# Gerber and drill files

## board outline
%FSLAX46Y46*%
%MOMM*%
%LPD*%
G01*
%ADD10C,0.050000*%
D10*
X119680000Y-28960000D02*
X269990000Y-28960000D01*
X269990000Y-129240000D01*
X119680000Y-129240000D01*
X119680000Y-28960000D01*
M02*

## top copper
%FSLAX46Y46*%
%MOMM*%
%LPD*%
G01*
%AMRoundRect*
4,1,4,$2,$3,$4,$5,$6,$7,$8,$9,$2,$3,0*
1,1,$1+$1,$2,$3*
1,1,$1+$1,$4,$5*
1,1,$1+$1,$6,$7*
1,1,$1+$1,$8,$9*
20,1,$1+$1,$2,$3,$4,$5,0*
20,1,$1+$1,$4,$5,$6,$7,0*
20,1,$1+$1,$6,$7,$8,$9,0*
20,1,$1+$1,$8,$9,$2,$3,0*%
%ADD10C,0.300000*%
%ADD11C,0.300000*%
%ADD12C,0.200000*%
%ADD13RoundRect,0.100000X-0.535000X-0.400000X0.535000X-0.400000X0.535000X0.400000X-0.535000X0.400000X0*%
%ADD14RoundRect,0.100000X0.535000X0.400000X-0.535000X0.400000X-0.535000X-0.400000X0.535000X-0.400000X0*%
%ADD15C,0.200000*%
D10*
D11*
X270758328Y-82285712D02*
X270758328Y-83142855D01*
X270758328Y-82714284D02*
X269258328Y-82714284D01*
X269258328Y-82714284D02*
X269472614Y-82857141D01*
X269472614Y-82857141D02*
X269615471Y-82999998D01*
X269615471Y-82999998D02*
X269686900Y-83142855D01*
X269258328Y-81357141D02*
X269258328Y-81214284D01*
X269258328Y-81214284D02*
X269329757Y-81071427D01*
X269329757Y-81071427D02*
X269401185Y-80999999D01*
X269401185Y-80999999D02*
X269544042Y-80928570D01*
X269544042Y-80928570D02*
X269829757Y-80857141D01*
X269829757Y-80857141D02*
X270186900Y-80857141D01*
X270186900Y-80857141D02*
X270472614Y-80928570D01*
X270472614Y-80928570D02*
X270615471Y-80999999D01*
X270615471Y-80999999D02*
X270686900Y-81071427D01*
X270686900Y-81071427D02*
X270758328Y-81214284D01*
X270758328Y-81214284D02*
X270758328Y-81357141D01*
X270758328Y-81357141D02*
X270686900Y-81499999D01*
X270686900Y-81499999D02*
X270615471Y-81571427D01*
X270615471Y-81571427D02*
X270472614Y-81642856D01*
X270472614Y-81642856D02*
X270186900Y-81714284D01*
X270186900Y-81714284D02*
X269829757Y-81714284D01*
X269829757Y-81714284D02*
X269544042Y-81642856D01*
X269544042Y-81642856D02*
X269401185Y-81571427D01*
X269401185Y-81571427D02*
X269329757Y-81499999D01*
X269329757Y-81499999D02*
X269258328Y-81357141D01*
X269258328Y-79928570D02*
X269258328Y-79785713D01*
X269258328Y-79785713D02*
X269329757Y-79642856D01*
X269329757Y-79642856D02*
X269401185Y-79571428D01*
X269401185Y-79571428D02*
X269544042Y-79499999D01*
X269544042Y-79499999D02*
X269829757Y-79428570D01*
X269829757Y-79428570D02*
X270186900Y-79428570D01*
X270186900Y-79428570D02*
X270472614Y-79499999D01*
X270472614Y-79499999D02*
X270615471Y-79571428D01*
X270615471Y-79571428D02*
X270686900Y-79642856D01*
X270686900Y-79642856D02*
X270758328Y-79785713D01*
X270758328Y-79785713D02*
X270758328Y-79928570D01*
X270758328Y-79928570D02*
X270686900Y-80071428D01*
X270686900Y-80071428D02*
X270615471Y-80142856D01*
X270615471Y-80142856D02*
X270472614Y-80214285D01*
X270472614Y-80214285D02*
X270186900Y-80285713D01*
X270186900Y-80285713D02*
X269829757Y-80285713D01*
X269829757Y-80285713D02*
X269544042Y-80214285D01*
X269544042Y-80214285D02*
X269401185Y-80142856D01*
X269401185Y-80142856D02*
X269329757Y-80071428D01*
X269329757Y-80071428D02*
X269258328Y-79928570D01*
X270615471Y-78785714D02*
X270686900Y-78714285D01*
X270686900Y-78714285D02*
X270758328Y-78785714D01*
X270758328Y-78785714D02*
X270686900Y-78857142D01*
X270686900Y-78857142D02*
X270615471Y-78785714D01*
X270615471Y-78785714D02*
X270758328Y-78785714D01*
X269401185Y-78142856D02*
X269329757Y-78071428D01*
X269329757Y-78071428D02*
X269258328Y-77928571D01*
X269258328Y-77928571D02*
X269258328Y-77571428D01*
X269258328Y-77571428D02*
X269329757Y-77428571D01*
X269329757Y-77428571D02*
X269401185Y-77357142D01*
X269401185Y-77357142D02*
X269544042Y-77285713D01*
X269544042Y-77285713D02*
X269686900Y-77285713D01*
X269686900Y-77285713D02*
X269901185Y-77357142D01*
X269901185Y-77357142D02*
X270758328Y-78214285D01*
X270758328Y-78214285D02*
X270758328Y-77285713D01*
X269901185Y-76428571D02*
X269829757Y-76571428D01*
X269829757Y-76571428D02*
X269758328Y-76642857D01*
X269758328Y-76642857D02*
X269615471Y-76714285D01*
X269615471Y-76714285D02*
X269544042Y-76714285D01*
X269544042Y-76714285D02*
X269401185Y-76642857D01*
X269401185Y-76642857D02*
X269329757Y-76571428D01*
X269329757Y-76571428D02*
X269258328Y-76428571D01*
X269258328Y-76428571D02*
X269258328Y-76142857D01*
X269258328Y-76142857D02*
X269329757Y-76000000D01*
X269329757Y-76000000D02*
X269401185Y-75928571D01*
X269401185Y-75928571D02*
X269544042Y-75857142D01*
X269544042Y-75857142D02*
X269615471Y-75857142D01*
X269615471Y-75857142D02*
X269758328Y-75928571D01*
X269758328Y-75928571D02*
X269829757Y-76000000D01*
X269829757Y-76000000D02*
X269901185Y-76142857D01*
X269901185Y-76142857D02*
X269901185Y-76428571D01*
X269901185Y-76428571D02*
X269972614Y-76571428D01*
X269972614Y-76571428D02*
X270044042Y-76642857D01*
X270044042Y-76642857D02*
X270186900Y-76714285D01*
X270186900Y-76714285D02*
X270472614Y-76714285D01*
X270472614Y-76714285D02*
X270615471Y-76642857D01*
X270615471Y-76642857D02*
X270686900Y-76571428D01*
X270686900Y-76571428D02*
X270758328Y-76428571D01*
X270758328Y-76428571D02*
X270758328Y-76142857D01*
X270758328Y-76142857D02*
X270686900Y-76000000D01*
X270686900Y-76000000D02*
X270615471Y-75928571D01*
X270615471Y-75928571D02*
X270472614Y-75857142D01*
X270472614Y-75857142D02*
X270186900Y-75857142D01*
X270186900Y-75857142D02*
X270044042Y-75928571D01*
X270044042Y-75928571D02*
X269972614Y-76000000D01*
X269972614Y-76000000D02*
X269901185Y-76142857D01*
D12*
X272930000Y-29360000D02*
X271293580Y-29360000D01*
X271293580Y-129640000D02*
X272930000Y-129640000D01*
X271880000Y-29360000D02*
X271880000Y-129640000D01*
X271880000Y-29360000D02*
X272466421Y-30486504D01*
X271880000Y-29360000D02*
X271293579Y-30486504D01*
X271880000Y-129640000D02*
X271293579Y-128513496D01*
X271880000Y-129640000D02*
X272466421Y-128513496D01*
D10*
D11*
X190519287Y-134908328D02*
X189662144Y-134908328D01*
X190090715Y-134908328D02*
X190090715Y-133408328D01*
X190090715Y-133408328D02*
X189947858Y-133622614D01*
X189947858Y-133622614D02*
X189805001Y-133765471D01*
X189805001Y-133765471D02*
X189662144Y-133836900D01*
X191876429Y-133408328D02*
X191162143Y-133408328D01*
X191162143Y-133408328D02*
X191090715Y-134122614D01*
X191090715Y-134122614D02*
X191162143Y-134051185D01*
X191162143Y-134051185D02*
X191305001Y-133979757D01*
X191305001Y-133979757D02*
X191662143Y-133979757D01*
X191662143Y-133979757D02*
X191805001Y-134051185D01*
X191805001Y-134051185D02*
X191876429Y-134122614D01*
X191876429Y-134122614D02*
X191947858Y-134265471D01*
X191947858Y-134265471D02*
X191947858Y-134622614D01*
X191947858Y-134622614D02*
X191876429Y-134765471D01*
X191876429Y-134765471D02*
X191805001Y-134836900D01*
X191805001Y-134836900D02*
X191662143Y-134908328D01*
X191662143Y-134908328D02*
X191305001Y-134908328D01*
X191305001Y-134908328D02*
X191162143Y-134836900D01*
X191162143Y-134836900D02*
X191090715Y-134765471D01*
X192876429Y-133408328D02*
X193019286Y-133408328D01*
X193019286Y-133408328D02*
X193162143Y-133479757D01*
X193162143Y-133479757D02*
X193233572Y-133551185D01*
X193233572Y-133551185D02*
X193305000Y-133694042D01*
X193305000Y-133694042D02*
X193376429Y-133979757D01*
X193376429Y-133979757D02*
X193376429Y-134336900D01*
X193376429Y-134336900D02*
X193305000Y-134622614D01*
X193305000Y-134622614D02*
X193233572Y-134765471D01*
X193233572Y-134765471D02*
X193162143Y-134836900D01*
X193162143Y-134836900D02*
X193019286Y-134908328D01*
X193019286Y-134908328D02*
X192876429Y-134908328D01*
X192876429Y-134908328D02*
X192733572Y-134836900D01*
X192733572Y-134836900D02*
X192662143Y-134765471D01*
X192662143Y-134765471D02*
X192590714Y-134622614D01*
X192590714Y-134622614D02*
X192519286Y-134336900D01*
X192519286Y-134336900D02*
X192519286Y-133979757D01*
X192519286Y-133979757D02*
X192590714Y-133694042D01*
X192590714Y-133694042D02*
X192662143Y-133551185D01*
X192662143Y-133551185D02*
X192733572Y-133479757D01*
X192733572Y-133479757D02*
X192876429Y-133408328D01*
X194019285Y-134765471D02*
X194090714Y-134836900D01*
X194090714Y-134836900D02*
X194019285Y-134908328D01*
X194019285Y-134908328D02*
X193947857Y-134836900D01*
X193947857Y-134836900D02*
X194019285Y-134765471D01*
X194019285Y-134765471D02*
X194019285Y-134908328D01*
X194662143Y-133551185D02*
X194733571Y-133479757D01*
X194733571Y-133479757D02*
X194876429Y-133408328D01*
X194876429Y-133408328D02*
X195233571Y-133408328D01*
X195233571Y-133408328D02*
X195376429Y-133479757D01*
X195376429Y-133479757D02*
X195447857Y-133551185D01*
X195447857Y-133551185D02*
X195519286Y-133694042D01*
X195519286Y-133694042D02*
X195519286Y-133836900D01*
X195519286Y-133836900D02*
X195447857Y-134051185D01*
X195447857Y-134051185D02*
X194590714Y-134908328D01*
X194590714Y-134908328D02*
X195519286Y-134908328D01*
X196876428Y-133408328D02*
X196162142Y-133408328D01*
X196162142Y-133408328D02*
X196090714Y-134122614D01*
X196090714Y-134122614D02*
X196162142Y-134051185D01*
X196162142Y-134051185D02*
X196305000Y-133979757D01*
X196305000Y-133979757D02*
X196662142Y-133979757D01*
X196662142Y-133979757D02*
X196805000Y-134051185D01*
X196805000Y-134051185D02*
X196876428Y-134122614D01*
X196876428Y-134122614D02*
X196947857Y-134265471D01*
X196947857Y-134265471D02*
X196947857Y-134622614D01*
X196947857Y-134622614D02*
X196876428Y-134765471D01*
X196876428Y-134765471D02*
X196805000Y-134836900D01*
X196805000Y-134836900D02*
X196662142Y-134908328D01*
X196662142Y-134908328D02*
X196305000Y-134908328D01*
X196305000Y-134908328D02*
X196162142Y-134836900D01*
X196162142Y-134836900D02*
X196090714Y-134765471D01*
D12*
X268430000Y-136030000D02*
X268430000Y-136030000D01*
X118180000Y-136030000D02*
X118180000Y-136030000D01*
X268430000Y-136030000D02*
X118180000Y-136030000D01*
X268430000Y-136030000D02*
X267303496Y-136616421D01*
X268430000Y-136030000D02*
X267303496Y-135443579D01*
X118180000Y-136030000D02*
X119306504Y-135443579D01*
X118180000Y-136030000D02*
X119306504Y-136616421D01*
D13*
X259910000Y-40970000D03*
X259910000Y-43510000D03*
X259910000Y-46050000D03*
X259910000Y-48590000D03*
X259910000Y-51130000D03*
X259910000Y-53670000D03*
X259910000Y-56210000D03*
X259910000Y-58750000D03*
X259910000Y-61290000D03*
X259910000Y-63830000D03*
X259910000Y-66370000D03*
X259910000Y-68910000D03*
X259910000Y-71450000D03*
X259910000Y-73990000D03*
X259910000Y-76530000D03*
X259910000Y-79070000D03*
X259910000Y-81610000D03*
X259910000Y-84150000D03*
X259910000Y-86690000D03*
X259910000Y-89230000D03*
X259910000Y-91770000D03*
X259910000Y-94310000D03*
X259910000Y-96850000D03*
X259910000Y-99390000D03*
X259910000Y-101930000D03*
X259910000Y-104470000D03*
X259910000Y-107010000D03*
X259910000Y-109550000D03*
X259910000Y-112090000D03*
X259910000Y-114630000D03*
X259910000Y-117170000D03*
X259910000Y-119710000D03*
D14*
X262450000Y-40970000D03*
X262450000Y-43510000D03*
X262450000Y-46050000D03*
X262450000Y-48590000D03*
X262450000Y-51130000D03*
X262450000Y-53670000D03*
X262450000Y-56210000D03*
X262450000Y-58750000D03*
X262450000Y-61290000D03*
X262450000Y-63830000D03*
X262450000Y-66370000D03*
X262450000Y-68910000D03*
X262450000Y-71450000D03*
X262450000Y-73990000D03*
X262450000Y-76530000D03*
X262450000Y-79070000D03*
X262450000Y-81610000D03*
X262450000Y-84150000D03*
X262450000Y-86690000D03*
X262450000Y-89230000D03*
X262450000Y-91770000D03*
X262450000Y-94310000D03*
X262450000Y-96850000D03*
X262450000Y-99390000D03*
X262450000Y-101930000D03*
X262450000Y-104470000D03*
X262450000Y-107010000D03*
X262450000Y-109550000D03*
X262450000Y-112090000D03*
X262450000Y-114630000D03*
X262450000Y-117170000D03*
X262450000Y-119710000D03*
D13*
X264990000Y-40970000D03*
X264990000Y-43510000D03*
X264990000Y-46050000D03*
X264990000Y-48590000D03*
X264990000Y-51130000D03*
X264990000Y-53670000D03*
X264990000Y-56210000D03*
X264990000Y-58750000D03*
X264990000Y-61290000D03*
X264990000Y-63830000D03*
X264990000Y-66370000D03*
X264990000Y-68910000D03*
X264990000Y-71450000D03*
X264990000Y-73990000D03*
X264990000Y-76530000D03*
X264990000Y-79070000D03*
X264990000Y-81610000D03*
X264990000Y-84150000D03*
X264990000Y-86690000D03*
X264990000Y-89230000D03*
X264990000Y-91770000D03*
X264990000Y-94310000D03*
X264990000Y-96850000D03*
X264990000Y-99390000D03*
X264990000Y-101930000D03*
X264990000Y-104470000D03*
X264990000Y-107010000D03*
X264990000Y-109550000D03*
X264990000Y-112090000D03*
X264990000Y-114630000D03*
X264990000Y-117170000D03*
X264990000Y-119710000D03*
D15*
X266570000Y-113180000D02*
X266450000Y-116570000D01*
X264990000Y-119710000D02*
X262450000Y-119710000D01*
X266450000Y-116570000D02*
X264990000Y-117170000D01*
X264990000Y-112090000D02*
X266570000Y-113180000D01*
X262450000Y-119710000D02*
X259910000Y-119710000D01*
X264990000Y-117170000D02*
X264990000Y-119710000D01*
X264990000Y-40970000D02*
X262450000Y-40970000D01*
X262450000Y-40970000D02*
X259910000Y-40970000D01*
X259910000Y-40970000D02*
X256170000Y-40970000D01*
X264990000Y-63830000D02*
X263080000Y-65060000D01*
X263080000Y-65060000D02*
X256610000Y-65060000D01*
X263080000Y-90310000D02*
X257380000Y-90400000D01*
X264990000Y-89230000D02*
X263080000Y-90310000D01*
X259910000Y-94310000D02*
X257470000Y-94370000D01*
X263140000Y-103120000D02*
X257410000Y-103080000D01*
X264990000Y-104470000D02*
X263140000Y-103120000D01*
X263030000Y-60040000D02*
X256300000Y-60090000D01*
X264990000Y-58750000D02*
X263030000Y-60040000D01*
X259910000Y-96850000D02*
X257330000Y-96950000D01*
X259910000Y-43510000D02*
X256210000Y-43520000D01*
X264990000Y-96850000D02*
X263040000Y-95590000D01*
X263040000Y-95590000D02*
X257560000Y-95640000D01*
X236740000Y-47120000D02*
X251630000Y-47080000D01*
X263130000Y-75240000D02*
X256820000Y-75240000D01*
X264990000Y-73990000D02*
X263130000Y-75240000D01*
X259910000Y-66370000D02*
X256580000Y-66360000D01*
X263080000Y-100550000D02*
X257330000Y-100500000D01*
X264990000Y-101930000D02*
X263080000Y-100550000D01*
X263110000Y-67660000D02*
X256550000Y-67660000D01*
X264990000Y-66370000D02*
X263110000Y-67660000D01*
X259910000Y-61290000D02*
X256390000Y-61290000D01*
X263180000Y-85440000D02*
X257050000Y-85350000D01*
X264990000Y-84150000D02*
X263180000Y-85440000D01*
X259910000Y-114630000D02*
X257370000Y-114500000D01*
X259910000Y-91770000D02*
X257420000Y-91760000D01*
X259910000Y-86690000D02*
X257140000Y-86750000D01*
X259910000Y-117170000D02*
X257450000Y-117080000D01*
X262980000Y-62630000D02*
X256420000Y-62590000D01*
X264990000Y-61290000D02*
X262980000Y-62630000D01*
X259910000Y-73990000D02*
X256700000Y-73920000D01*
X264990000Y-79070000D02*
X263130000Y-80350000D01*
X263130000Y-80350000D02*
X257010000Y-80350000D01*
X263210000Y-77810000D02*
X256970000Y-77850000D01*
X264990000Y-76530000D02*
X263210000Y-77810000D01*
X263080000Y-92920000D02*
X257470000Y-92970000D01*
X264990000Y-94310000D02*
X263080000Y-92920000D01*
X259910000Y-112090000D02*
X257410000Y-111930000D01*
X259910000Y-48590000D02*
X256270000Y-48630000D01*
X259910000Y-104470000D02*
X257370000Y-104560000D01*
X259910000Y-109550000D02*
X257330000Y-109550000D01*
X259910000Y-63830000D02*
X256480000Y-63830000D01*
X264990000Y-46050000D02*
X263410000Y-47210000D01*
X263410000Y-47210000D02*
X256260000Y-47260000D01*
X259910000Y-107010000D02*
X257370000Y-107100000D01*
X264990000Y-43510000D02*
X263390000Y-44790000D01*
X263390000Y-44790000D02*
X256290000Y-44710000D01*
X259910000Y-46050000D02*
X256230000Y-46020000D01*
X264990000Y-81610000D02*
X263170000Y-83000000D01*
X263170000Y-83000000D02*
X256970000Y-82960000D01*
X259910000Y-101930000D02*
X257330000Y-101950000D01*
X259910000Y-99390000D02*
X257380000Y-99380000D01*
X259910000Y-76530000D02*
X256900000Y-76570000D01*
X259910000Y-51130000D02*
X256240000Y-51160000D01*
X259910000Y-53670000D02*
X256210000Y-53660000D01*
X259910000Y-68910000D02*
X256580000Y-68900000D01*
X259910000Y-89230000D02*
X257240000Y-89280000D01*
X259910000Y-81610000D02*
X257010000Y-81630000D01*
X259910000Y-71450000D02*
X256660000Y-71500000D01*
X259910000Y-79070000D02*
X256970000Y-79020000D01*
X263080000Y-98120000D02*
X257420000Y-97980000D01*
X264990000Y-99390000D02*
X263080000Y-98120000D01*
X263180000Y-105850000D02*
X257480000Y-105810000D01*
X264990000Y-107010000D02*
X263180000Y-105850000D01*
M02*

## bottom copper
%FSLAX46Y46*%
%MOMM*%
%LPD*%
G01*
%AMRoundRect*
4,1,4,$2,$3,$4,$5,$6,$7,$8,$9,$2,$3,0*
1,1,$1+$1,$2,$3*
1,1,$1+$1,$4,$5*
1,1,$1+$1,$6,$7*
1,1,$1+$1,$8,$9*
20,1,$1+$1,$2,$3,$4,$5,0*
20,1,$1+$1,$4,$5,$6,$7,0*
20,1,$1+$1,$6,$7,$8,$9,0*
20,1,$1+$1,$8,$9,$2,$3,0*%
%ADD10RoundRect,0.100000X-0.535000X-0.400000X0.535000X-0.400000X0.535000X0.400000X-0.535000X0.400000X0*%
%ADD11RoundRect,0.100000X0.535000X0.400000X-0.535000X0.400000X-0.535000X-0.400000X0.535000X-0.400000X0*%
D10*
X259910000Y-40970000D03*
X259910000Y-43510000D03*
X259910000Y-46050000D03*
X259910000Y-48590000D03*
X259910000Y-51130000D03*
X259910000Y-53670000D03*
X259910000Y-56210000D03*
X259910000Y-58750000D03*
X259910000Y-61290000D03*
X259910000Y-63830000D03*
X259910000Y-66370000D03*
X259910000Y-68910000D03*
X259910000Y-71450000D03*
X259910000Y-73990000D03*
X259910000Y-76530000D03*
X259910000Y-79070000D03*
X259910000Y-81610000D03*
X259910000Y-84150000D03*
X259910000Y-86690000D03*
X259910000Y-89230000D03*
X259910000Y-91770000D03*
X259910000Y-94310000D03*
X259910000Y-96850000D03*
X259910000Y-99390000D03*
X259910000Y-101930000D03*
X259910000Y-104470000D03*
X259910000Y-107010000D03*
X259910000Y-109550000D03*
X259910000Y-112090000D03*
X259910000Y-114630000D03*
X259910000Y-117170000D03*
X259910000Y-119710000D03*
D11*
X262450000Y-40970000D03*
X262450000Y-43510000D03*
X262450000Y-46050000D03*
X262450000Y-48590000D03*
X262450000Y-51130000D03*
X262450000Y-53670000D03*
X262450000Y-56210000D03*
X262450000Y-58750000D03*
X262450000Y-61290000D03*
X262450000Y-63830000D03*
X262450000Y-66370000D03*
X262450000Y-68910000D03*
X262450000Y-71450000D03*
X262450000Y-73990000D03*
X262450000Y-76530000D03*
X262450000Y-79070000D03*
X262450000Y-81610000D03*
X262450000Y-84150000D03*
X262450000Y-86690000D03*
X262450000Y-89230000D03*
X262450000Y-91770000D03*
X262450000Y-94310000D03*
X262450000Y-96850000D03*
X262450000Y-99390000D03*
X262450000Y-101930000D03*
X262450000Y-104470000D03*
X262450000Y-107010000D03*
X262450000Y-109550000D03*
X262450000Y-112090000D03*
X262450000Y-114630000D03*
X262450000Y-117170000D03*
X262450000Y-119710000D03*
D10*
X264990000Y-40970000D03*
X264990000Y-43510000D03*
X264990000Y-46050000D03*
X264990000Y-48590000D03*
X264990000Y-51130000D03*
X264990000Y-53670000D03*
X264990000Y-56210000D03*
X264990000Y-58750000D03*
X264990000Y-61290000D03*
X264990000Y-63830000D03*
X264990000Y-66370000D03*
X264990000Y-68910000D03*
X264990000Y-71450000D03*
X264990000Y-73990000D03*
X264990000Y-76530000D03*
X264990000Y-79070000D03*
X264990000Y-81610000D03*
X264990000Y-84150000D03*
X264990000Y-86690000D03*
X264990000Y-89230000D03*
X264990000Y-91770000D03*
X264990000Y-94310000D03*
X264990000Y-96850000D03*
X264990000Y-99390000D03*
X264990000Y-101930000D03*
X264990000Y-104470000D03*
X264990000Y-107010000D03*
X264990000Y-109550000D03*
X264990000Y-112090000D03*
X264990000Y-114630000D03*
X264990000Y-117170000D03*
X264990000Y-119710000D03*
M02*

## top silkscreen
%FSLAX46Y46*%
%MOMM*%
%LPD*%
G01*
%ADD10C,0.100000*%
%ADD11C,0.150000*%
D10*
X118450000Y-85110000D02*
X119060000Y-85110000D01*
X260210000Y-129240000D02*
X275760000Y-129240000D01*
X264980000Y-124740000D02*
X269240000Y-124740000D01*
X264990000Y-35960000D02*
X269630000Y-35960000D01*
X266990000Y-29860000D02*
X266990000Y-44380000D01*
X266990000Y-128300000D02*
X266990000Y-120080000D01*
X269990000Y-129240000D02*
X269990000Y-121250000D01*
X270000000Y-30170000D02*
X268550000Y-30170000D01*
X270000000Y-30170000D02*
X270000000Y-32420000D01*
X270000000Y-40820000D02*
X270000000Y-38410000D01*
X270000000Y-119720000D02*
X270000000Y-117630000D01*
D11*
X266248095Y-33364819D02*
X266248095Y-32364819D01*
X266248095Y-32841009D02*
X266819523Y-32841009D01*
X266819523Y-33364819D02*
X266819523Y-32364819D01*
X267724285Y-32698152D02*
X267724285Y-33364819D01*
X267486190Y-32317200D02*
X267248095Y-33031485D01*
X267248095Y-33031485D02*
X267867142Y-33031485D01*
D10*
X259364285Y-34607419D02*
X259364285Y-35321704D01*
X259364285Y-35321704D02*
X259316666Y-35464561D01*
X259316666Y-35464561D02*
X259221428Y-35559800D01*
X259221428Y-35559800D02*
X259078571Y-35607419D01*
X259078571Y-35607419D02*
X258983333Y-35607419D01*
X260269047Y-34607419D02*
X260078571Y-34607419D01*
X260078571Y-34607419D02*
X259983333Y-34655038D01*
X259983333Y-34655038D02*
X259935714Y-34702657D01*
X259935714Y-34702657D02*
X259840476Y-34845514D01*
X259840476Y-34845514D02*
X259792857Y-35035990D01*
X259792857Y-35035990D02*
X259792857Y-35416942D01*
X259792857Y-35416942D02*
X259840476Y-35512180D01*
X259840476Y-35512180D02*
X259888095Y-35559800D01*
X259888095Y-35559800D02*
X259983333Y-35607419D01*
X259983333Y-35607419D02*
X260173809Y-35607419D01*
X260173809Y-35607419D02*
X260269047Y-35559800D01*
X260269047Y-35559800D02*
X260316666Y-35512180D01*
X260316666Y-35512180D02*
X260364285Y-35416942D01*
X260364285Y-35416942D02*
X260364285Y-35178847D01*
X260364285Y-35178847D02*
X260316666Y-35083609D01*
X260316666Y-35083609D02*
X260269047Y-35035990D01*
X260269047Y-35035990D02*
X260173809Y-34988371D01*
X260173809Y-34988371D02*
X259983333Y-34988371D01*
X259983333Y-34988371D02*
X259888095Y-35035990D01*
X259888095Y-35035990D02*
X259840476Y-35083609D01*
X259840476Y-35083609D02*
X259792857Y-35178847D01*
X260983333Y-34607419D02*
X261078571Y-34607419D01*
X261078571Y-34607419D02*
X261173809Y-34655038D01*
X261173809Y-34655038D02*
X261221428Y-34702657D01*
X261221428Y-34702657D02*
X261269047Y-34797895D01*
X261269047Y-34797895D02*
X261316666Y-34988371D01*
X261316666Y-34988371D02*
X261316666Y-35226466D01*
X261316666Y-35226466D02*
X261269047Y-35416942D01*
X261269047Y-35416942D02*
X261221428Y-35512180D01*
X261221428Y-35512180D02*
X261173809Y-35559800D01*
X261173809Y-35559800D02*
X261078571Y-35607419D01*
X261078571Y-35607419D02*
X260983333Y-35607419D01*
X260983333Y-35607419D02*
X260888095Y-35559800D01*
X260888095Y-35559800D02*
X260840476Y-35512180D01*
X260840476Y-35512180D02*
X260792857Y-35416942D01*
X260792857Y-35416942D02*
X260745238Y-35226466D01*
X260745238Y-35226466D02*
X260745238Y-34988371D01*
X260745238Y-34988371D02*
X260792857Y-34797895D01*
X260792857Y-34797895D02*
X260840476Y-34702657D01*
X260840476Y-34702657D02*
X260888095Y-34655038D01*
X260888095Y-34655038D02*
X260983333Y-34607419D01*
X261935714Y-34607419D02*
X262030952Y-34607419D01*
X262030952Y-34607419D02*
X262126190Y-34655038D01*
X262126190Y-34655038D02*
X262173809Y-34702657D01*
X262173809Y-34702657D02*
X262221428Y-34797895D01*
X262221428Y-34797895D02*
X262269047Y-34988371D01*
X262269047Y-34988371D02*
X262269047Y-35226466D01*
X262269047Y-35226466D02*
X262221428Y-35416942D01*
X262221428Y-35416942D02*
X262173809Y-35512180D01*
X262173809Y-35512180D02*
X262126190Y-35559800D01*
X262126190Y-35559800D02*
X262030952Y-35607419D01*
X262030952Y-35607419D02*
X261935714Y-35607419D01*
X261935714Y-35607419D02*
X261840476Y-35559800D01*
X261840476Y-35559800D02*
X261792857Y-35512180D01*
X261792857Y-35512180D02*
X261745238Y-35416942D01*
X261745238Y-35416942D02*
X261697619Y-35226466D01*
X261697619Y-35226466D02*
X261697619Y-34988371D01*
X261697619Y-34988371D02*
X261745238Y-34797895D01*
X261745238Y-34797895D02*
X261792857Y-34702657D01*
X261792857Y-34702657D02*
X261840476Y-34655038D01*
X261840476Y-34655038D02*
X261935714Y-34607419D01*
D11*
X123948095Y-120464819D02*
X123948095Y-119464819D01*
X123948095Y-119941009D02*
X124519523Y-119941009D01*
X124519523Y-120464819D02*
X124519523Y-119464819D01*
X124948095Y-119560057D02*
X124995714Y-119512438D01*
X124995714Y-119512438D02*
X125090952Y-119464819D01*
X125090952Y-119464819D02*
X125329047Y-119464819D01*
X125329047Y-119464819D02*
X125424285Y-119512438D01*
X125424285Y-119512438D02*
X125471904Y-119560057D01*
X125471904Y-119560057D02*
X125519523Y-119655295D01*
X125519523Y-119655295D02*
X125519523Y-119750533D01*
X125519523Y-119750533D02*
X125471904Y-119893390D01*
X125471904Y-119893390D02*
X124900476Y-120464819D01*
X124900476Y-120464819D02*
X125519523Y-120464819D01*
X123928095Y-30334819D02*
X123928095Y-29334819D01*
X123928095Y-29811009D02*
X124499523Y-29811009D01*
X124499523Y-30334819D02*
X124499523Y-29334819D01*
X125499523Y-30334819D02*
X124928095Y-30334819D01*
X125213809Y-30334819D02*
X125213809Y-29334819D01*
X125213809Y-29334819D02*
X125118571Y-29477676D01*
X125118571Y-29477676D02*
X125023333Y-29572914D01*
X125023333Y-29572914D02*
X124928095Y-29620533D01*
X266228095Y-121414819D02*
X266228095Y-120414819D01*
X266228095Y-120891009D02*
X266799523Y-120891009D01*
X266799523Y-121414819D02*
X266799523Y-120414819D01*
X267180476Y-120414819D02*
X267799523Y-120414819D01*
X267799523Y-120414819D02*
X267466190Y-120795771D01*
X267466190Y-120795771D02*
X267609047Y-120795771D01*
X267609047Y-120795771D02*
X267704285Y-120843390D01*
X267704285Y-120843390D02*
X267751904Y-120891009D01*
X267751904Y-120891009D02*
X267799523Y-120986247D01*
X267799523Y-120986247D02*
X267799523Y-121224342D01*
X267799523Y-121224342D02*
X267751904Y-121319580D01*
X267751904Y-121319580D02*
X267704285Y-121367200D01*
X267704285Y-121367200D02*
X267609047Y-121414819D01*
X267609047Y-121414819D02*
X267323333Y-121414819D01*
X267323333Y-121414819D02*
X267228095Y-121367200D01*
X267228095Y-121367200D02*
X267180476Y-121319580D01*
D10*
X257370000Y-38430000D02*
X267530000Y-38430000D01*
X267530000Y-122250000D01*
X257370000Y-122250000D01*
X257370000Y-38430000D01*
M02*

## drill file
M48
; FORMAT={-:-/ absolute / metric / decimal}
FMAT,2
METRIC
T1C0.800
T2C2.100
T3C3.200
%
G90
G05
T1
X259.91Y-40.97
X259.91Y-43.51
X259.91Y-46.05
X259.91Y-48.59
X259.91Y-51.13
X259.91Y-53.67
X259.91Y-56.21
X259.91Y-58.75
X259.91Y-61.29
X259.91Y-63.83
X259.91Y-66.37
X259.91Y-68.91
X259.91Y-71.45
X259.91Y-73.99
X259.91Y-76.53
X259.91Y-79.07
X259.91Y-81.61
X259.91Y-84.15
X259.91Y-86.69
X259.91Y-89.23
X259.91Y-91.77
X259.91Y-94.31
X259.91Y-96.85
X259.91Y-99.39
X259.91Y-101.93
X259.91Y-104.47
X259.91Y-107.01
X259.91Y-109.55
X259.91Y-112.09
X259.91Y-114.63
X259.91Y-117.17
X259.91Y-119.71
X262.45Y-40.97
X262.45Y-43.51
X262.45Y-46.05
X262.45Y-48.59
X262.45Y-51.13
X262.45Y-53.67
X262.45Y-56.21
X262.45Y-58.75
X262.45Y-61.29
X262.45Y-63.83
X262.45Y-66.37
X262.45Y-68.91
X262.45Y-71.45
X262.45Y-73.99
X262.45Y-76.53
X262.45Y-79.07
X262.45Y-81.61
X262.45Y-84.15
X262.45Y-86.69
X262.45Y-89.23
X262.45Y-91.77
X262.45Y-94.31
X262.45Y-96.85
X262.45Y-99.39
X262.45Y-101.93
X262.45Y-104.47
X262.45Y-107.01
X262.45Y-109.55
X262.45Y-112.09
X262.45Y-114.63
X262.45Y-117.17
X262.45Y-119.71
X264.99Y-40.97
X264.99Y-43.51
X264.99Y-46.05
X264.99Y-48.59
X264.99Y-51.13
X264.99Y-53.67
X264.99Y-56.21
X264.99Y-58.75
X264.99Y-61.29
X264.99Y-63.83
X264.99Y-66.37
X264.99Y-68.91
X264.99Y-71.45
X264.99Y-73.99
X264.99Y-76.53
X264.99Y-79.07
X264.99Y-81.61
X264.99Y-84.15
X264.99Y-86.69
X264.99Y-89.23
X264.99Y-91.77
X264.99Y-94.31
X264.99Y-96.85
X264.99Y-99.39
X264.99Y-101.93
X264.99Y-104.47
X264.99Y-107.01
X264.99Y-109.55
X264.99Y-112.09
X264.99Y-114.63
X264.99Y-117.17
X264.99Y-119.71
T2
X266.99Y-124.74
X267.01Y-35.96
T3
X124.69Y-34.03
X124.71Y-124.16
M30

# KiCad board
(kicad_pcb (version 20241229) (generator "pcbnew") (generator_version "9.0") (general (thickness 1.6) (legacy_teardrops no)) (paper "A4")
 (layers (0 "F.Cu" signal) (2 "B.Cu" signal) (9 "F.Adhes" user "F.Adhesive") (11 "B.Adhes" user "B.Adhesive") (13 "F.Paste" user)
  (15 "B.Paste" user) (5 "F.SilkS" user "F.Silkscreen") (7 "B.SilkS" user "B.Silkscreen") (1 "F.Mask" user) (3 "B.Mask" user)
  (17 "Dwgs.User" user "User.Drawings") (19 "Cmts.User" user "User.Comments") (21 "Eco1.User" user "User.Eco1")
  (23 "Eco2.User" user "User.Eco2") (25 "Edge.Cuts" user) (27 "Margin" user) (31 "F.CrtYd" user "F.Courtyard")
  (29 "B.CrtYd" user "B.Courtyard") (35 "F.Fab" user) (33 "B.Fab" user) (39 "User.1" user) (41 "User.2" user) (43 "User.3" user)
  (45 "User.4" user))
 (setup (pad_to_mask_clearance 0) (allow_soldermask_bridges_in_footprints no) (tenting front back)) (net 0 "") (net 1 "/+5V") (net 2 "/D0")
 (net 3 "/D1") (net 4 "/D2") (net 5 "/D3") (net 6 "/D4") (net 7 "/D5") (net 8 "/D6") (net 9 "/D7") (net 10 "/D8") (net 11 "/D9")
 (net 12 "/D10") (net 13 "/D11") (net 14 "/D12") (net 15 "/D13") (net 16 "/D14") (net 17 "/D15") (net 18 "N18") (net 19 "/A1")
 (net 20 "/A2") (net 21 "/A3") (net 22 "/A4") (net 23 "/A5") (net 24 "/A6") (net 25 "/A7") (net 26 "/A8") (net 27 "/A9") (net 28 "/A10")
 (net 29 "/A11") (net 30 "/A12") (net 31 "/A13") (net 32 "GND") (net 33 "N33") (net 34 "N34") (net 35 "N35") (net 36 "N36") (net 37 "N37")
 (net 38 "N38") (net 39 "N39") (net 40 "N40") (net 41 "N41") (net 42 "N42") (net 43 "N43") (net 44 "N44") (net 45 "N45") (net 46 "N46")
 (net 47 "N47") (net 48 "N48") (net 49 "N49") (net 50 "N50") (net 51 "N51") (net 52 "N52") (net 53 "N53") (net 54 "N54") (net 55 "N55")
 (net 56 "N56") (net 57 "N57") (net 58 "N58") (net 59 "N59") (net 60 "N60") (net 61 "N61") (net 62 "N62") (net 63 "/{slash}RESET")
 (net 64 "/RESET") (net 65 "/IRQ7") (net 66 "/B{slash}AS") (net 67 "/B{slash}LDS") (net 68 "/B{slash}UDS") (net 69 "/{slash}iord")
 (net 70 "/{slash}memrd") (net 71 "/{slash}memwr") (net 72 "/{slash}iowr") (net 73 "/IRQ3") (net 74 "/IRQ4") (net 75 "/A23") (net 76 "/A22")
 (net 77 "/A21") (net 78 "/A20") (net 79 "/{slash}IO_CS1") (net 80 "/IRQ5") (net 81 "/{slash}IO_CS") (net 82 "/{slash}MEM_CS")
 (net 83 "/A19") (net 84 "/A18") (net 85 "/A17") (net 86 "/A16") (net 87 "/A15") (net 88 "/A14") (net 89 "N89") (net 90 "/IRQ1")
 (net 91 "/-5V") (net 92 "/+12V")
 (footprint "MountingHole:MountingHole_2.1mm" (layer "F.Cu") (at 267.01 35.96)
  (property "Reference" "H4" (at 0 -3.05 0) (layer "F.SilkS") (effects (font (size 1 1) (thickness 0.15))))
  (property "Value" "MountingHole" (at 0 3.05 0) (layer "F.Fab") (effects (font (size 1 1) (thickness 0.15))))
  (pad "" np_thru_hole circle (at 0 0) (size 2.1 2.1) (drill 2.1) (layers "*.Cu" "*.Mask")))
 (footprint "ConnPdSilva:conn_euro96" (layer "F.Cu") (at 262.45 35.89)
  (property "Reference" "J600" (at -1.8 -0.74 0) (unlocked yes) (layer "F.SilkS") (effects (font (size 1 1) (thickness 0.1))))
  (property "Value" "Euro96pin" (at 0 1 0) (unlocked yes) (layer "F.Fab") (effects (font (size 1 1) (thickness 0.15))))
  (fp_rect (start -5.08 2.54) (end 5.08 86.36) (stroke (width 0.1) (type default)) (fill no) (layer "F.SilkS"))
  (pad "1" thru_hole roundrect (at -2.54 5.08) (size 1.27 1) (drill 0.8) (layers "*.Cu" "*.Mask") (remove_unused_layers no)
   (roundrect_rratio 0.1) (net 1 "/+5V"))
  (pad "2" thru_hole roundrect (at -2.54 7.62) (size 1.27 1) (drill 0.8) (layers "*.Cu" "*.Mask") (remove_unused_layers no)
   (roundrect_rratio 0.1) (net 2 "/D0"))
  (pad "3" thru_hole roundrect (at -2.54 10.16) (size 1.27 1) (drill 0.8) (layers "*.Cu" "*.Mask") (remove_unused_layers no)
   (roundrect_rratio 0.1) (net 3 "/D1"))
  (pad "4" thru_hole roundrect (at -2.54 12.7) (size 1.27 1) (drill 0.8) (layers "*.Cu" "*.Mask") (remove_unused_layers no)
   (roundrect_rratio 0.1) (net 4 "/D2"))
  (pad "5" thru_hole roundrect (at -2.54 15.24) (size 1.27 1) (drill 0.8) (layers "*.Cu" "*.Mask") (remove_unused_layers no)
   (roundrect_rratio 0.1) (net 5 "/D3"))
  (pad "6" thru_hole roundrect (at -2.54 17.78) (size 1.27 1) (drill 0.8) (layers "*.Cu" "*.Mask") (remove_unused_layers no)
   (roundrect_rratio 0.1) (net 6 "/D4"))
  (pad "7" thru_hole roundrect (at -2.54 20.32) (size 1.27 1) (drill 0.8) (layers "*.Cu" "*.Mask") (remove_unused_layers no)
   (roundrect_rratio 0.1) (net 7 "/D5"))
  (pad "8" thru_hole roundrect (at -2.54 22.86) (size 1.27 1) (drill 0.8) (layers "*.Cu" "*.Mask") (remove_unused_layers no)
   (roundrect_rratio 0.1) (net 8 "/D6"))
  (pad "9" thru_hole roundrect (at -2.54 25.4) (size 1.27 1) (drill 0.8) (layers "*.Cu" "*.Mask") (remove_unused_layers no)
   (roundrect_rratio 0.1) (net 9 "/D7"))
  (pad "10" thru_hole roundrect (at -2.54 27.94) (size 1.27 1) (drill 0.8) (layers "*.Cu" "*.Mask") (remove_unused_layers no)
   (roundrect_rratio 0.1) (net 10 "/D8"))
  (pad "11" thru_hole roundrect (at -2.54 30.48) (size 1.27 1) (drill 0.8) (layers "*.Cu" "*.Mask") (remove_unused_layers no)
   (roundrect_rratio 0.1) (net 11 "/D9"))
  (pad "12" thru_hole roundrect (at -2.54 33.02) (size 1.27 1) (drill 0.8) (layers "*.Cu" "*.Mask") (remove_unused_layers no)
   (roundrect_rratio 0.1) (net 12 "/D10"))
  (pad "13" thru_hole roundrect (at -2.54 35.56) (size 1.27 1) (drill 0.8) (layers "*.Cu" "*.Mask") (remove_unused_layers no)
   (roundrect_rratio 0.1) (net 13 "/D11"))
  (pad "14" thru_hole roundrect (at -2.54 38.1) (size 1.27 1) (drill 0.8) (layers "*.Cu" "*.Mask") (remove_unused_layers no)
   (roundrect_rratio 0.1) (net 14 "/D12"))
  (pad "15" thru_hole roundrect (at -2.54 40.64) (size 1.27 1) (drill 0.8) (layers "*.Cu" "*.Mask") (remove_unused_layers no)
   (roundrect_rratio 0.1) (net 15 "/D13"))
  (pad "16" thru_hole roundrect (at -2.54 43.18) (size 1.27 1) (drill 0.8) (layers "*.Cu" "*.Mask") (remove_unused_layers no)
   (roundrect_rratio 0.1) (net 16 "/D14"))
  (pad "17" thru_hole roundrect (at -2.54 45.72) (size 1.27 1) (drill 0.8) (layers "*.Cu" "*.Mask") (remove_unused_layers no)
   (roundrect_rratio 0.1) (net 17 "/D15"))
  (pad "18" thru_hole roundrect (at -2.54 48.26) (size 1.27 1) (drill 0.8) (layers "*.Cu" "*.Mask") (remove_unused_layers no)
   (roundrect_rratio 0.1) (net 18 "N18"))
  (pad "19" thru_hole roundrect (at -2.54 50.8) (size 1.27 1) (drill 0.8) (layers "*.Cu" "*.Mask") (remove_unused_layers no)
   (roundrect_rratio 0.1) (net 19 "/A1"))
  (pad "20" thru_hole roundrect (at -2.54 53.34) (size 1.27 1) (drill 0.8) (layers "*.Cu" "*.Mask") (remove_unused_layers no)
   (roundrect_rratio 0.1) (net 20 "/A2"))
  (pad "21" thru_hole roundrect (at -2.54 55.88) (size 1.27 1) (drill 0.8) (layers "*.Cu" "*.Mask") (remove_unused_layers no)
   (roundrect_rratio 0.1) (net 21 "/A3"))
  (pad "22" thru_hole roundrect (at -2.54 58.42) (size 1.27 1) (drill 0.8) (layers "*.Cu" "*.Mask") (remove_unused_layers no)
   (roundrect_rratio 0.1) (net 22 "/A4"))
  (pad "23" thru_hole roundrect (at -2.54 60.96) (size 1.27 1) (drill 0.8) (layers "*.Cu" "*.Mask") (remove_unused_layers no)
   (roundrect_rratio 0.1) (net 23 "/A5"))
  (pad "24" thru_hole roundrect (at -2.54 63.5) (size 1.27 1) (drill 0.8) (layers "*.Cu" "*.Mask") (remove_unused_layers no)
   (roundrect_rratio 0.1) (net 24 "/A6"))
  (pad "25" thru_hole roundrect (at -2.54 66.04) (size 1.27 1) (drill 0.8) (layers "*.Cu" "*.Mask") (remove_unused_layers no)
   (roundrect_rratio 0.1) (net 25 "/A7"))
  (pad "26" thru_hole roundrect (at -2.54 68.58) (size 1.27 1) (drill 0.8) (layers "*.Cu" "*.Mask") (remove_unused_layers no)
   (roundrect_rratio 0.1) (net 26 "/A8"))
  (pad "27" thru_hole roundrect (at -2.54 71.12) (size 1.27 1) (drill 0.8) (layers "*.Cu" "*.Mask") (remove_unused_layers no)
   (roundrect_rratio 0.1) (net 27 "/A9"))
  (pad "28" thru_hole roundrect (at -2.54 73.66) (size 1.27 1) (drill 0.8) (layers "*.Cu" "*.Mask") (remove_unused_layers no)
   (roundrect_rratio 0.1) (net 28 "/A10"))
  (pad "29" thru_hole roundrect (at -2.54 76.2) (size 1.27 1) (drill 0.8) (layers "*.Cu" "*.Mask") (remove_unused_layers no)
   (roundrect_rratio 0.1) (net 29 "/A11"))
  (pad "30" thru_hole roundrect (at -2.54 78.74) (size 1.27 1) (drill 0.8) (layers "*.Cu" "*.Mask") (remove_unused_layers no)
   (roundrect_rratio 0.1) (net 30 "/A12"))
  (pad "31" thru_hole roundrect (at -2.54 81.28) (size 1.27 1) (drill 0.8) (layers "*.Cu" "*.Mask") (remove_unused_layers no)
   (roundrect_rratio 0.1) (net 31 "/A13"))
  (pad "32" thru_hole roundrect (at -2.54 83.82) (size 1.27 1) (drill 0.8) (layers "*.Cu" "*.Mask") (remove_unused_layers no)
   (roundrect_rratio 0.1) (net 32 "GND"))
  (pad "33" thru_hole roundrect (at 0 5.08 180) (size 1.27 1) (drill 0.8) (layers "*.Cu" "*.Mask") (remove_unused_layers no)
   (roundrect_rratio 0.1) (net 1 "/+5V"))
  (pad "34" thru_hole roundrect (at 0 7.62 180) (size 1.27 1) (drill 0.8) (layers "*.Cu" "*.Mask") (remove_unused_layers no)
   (roundrect_rratio 0.1) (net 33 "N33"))
  (pad "35" thru_hole roundrect (at 0 10.16 180) (size 1.27 1) (drill 0.8) (layers "*.Cu" "*.Mask") (remove_unused_layers no)
   (roundrect_rratio 0.1) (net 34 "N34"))
  (pad "36" thru_hole roundrect (at 0 12.7 180) (size 1.27 1) (drill 0.8) (layers "*.Cu" "*.Mask") (remove_unused_layers no)
   (roundrect_rratio 0.1) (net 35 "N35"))
  (pad "37" thru_hole roundrect (at 0 15.24 180) (size 1.27 1) (drill 0.8) (layers "*.Cu" "*.Mask") (remove_unused_layers no)
   (roundrect_rratio 0.1) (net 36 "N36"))
  (pad "38" thru_hole roundrect (at 0 17.78 180) (size 1.27 1) (drill 0.8) (layers "*.Cu" "*.Mask") (remove_unused_layers no)
   (roundrect_rratio 0.1) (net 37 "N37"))
  (pad "39" thru_hole roundrect (at 0 20.32 180) (size 1.27 1) (drill 0.8) (layers "*.Cu" "*.Mask") (remove_unused_layers no)
   (roundrect_rratio 0.1) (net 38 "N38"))
  (pad "40" thru_hole roundrect (at 0 22.86 180) (size 1.27 1) (drill 0.8) (layers "*.Cu" "*.Mask") (remove_unused_layers no)
   (roundrect_rratio 0.1) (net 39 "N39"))
  (pad "41" thru_hole roundrect (at 0 25.4 180) (size 1.27 1) (drill 0.8) (layers "*.Cu" "*.Mask") (remove_unused_layers no)
   (roundrect_rratio 0.1) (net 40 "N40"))
  (pad "42" thru_hole roundrect (at 0 27.94 180) (size 1.27 1) (drill 0.8) (layers "*.Cu" "*.Mask") (remove_unused_layers no)
   (roundrect_rratio 0.1) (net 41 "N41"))
  (pad "43" thru_hole roundrect (at 0 30.48 180) (size 1.27 1) (drill 0.8) (layers "*.Cu" "*.Mask") (remove_unused_layers no)
   (roundrect_rratio 0.1) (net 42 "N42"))
  (pad "44" thru_hole roundrect (at 0 33.02 180) (size 1.27 1) (drill 0.8) (layers "*.Cu" "*.Mask") (remove_unused_layers no)
   (roundrect_rratio 0.1) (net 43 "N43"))
  (pad "45" thru_hole roundrect (at 0 35.56 180) (size 1.27 1) (drill 0.8) (layers "*.Cu" "*.Mask") (remove_unused_layers no)
   (roundrect_rratio 0.1) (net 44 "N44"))
  (pad "46" thru_hole roundrect (at 0 38.1 180) (size 1.27 1) (drill 0.8) (layers "*.Cu" "*.Mask") (remove_unused_layers no)
   (roundrect_rratio 0.1) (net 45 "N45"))
  (pad "47" thru_hole roundrect (at 0 40.64 180) (size 1.27 1) (drill 0.8) (layers "*.Cu" "*.Mask") (remove_unused_layers no)
   (roundrect_rratio 0.1) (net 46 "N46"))
  (pad "48" thru_hole roundrect (at 0 43.18 180) (size 1.27 1) (drill 0.8) (layers "*.Cu" "*.Mask") (remove_unused_layers no)
   (roundrect_rratio 0.1) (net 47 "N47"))
  (pad "49" thru_hole roundrect (at 0 45.72 180) (size 1.27 1) (drill 0.8) (layers "*.Cu" "*.Mask") (remove_unused_layers no)
   (roundrect_rratio 0.1) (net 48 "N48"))
  (pad "50" thru_hole roundrect (at 0 48.26 180) (size 1.27 1) (drill 0.8) (layers "*.Cu" "*.Mask") (remove_unused_layers no)
   (roundrect_rratio 0.1) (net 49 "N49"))
  (pad "51" thru_hole roundrect (at 0 50.8 180) (size 1.27 1) (drill 0.8) (layers "*.Cu" "*.Mask") (remove_unused_layers no)
   (roundrect_rratio 0.1) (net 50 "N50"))
  (pad "52" thru_hole roundrect (at 0 53.34 180) (size 1.27 1) (drill 0.8) (layers "*.Cu" "*.Mask") (remove_unused_layers no)
   (roundrect_rratio 0.1) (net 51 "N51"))
  (pad "53" thru_hole roundrect (at 0 55.88 180) (size 1.27 1) (drill 0.8) (layers "*.Cu" "*.Mask") (remove_unused_layers no)
   (roundrect_rratio 0.1) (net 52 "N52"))
  (pad "54" thru_hole roundrect (at 0 58.42 180) (size 1.27 1) (drill 0.8) (layers "*.Cu" "*.Mask") (remove_unused_layers no)
   (roundrect_rratio 0.1) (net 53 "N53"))
  (pad "55" thru_hole roundrect (at 0 60.96 180) (size 1.27 1) (drill 0.8) (layers "*.Cu" "*.Mask") (remove_unused_layers no)
   (roundrect_rratio 0.1) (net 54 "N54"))
  (pad "56" thru_hole roundrect (at 0 63.5 180) (size 1.27 1) (drill 0.8) (layers "*.Cu" "*.Mask") (remove_unused_layers no)
   (roundrect_rratio 0.1) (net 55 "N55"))
  (pad "57" thru_hole roundrect (at 0 66.04 180) (size 1.27 1) (drill 0.8) (layers "*.Cu" "*.Mask") (remove_unused_layers no)
   (roundrect_rratio 0.1) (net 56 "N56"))
  (pad "58" thru_hole roundrect (at 0 68.58 180) (size 1.27 1) (drill 0.8) (layers "*.Cu" "*.Mask") (remove_unused_layers no)
   (roundrect_rratio 0.1) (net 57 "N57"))
  (pad "59" thru_hole roundrect (at 0 71.12 180) (size 1.27 1) (drill 0.8) (layers "*.Cu" "*.Mask") (remove_unused_layers no)
   (roundrect_rratio 0.1) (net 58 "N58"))
  (pad "60" thru_hole roundrect (at 0 73.66 180) (size 1.27 1) (drill 0.8) (layers "*.Cu" "*.Mask") (remove_unused_layers no)
   (roundrect_rratio 0.1) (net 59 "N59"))
  (pad "61" thru_hole roundrect (at 0 76.2 180) (size 1.27 1) (drill 0.8) (layers "*.Cu" "*.Mask") (remove_unused_layers no)
   (roundrect_rratio 0.1) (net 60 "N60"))
  (pad "62" thru_hole roundrect (at 0 78.74 180) (size 1.27 1) (drill 0.8) (layers "*.Cu" "*.Mask") (remove_unused_layers no)
   (roundrect_rratio 0.1) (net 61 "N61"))
  (pad "63" thru_hole roundrect (at 0 81.28 180) (size 1.27 1) (drill 0.8) (layers "*.Cu" "*.Mask") (remove_unused_layers no)
   (roundrect_rratio 0.1) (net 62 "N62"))
  (pad "64" thru_hole roundrect (at 0 83.82 180) (size 1.27 1) (drill 0.8) (layers "*.Cu" "*.Mask") (remove_unused_layers no)
   (roundrect_rratio 0.1) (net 32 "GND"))
  (pad "65" thru_hole roundrect (at 2.54 5.08) (size 1.27 1) (drill 0.8) (layers "*.Cu" "*.Mask") (remove_unused_layers no)
   (roundrect_rratio 0.1) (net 1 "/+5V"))
  (pad "66" thru_hole roundrect (at 2.54 7.62) (size 1.27 1) (drill 0.8) (layers "*.Cu" "*.Mask") (remove_unused_layers no)
   (roundrect_rratio 0.1) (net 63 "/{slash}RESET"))
  (pad "67" thru_hole roundrect (at 2.54 10.16) (size 1.27 1) (drill 0.8) (layers "*.Cu" "*.Mask") (remove_unused_layers no)
   (roundrect_rratio 0.1) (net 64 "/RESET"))
  (pad "68" thru_hole roundrect (at 2.54 12.7) (size 1.27 1) (drill 0.8) (layers "*.Cu" "*.Mask") (remove_unused_layers no)
   (roundrect_rratio 0.1) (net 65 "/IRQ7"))
  (pad "69" thru_hole roundrect (at 2.54 15.24) (size 1.27 1) (drill 0.8) (layers "*.Cu" "*.Mask") (remove_unused_layers no)
   (roundrect_rratio 0.1) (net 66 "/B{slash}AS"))
  (pad "70" thru_hole roundrect (at 2.54 17.78) (size 1.27 1) (drill 0.8) (layers "*.Cu" "*.Mask") (remove_unused_layers no)
   (roundrect_rratio 0.1) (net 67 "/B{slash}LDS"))
  (pad "71" thru_hole roundrect (at 2.54 20.32) (size 1.27 1) (drill 0.8) (layers "*.Cu" "*.Mask") (remove_unused_layers no)
   (roundrect_rratio 0.1) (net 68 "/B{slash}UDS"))
  (pad "72" thru_hole roundrect (at 2.54 22.86) (size 1.27 1) (drill 0.8) (layers "*.Cu" "*.Mask") (remove_unused_layers no)
   (roundrect_rratio 0.1) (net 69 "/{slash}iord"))
  (pad "73" thru_hole roundrect (at 2.54 25.4) (size 1.27 1) (drill 0.8) (layers "*.Cu" "*.Mask") (remove_unused_layers no)
   (roundrect_rratio 0.1) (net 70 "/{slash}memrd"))
  (pad "74" thru_hole roundrect (at 2.54 27.94) (size 1.27 1) (drill 0.8) (layers "*.Cu" "*.Mask") (remove_unused_layers no)
   (roundrect_rratio 0.1) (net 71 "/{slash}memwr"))
  (pad "75" thru_hole roundrect (at 2.54 30.48) (size 1.27 1) (drill 0.8) (layers "*.Cu" "*.Mask") (remove_unused_layers no)
   (roundrect_rratio 0.1) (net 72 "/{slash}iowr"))
  (pad "76" thru_hole roundrect (at 2.54 33.02) (size 1.27 1) (drill 0.8) (layers "*.Cu" "*.Mask") (remove_unused_layers no)
   (roundrect_rratio 0.1) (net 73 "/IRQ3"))
  (pad "77" thru_hole roundrect (at 2.54 35.56) (size 1.27 1) (drill 0.8) (layers "*.Cu" "*.Mask") (remove_unused_layers no)
   (roundrect_rratio 0.1) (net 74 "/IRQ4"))
  (pad "78" thru_hole roundrect (at 2.54 38.1) (size 1.27 1) (drill 0.8) (layers "*.Cu" "*.Mask") (remove_unused_layers no)
   (roundrect_rratio 0.1) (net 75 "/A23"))
  (pad "79" thru_hole roundrect (at 2.54 40.64) (size 1.27 1) (drill 0.8) (layers "*.Cu" "*.Mask") (remove_unused_layers no)
   (roundrect_rratio 0.1) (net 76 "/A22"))
  (pad "80" thru_hole roundrect (at 2.54 43.18) (size 1.27 1) (drill 0.8) (layers "*.Cu" "*.Mask") (remove_unused_layers no)
   (roundrect_rratio 0.1) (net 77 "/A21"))
  (pad "81" thru_hole roundrect (at 2.54 45.72) (size 1.27 1) (drill 0.8) (layers "*.Cu" "*.Mask") (remove_unused_layers no)
   (roundrect_rratio 0.1) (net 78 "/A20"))
  (pad "82" thru_hole roundrect (at 2.54 48.26) (size 1.27 1) (drill 0.8) (layers "*.Cu" "*.Mask") (remove_unused_layers no)
   (roundrect_rratio 0.1) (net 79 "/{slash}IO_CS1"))
  (pad "83" thru_hole roundrect (at 2.54 50.8) (size 1.27 1) (drill 0.8) (layers "*.Cu" "*.Mask") (remove_unused_layers no)
   (roundrect_rratio 0.1) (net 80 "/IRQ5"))
  (pad "84" thru_hole roundrect (at 2.54 53.34) (size 1.27 1) (drill 0.8) (layers "*.Cu" "*.Mask") (remove_unused_layers no)
   (roundrect_rratio 0.1) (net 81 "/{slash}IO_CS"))
  (pad "85" thru_hole roundrect (at 2.54 55.88) (size 1.27 1) (drill 0.8) (layers "*.Cu" "*.Mask") (remove_unused_layers no)
   (roundrect_rratio 0.1) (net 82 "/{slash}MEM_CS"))
  (pad "86" thru_hole roundrect (at 2.54 58.42) (size 1.27 1) (drill 0.8) (layers "*.Cu" "*.Mask") (remove_unused_layers no)
   (roundrect_rratio 0.1) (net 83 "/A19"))
  (pad "87" thru_hole roundrect (at 2.54 60.96) (size 1.27 1) (drill 0.8) (layers "*.Cu" "*.Mask") (remove_unused_layers no)
   (roundrect_rratio 0.1) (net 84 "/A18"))
  (pad "88" thru_hole roundrect (at 2.54 63.5) (size 1.27 1) (drill 0.8) (layers "*.Cu" "*.Mask") (remove_unused_layers no)
   (roundrect_rratio 0.1) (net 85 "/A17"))
  (pad "89" thru_hole roundrect (at 2.54 66.04) (size 1.27 1) (drill 0.8) (layers "*.Cu" "*.Mask") (remove_unused_layers no)
   (roundrect_rratio 0.1) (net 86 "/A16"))
  (pad "90" thru_hole roundrect (at 2.54 68.58) (size 1.27 1) (drill 0.8) (layers "*.Cu" "*.Mask") (remove_unused_layers no)
   (roundrect_rratio 0.1) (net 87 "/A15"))
  (pad "91" thru_hole roundrect (at 2.54 71.12) (size 1.27 1) (drill 0.8) (layers "*.Cu" "*.Mask") (remove_unused_layers no)
   (roundrect_rratio 0.1) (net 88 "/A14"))
  (pad "92" thru_hole roundrect (at 2.54 73.66) (size 1.27 1) (drill 0.8) (layers "*.Cu" "*.Mask") (remove_unused_layers no)
   (roundrect_rratio 0.1) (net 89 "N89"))
  (pad "93" thru_hole roundrect (at 2.54 76.2) (size 1.27 1) (drill 0.8) (layers "*.Cu" "*.Mask") (remove_unused_layers no)
   (roundrect_rratio 0.1) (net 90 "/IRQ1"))
  (pad "94" thru_hole roundrect (at 2.54 78.74) (size 1.27 1) (drill 0.8) (layers "*.Cu" "*.Mask") (remove_unused_layers no)
   (roundrect_rratio 0.1) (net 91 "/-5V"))
  (pad "95" thru_hole roundrect (at 2.54 81.28) (size 1.27 1) (drill 0.8) (layers "*.Cu" "*.Mask") (remove_unused_layers no)
   (roundrect_rratio 0.1) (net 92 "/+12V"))
  (pad "96" thru_hole roundrect (at 2.54 83.82) (size 1.27 1) (drill 0.8) (layers "*.Cu" "*.Mask") (remove_unused_layers no)
   (roundrect_rratio 0.1) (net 32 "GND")))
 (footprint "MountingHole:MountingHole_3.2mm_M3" (layer "F.Cu") (at 124.71 124.16)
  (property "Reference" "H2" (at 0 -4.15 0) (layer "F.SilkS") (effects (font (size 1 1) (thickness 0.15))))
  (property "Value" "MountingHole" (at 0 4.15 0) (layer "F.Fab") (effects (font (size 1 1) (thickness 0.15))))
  (pad "" np_thru_hole circle (at 0 0) (size 3.2 3.2) (drill 3.2) (layers "*.Cu" "*.Mask")))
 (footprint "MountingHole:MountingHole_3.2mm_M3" (layer "F.Cu") (at 124.69 34.03)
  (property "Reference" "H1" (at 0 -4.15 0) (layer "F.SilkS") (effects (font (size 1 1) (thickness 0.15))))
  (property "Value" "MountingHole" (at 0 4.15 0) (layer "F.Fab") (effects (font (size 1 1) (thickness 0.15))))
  (pad "" np_thru_hole circle (at 0 0) (size 3.2 3.2) (drill 3.2) (layers "*.Cu" "*.Mask")))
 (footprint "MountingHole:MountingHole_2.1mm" (layer "F.Cu") (at 266.99 124.74)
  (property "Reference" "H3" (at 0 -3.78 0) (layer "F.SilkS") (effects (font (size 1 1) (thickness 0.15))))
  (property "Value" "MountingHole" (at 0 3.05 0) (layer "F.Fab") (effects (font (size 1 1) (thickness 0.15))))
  (pad "" np_thru_hole circle (at 0 0) (size 2.1 2.1) (drill 2.1) (layers "*.Cu" "*.Mask")))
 (gr_line (start 118.45 85.11) (end 119.06 85.11) (stroke (width 0.1) (type default)) (layer "F.SilkS"))
 (gr_line (start 260.21 129.24) (end 275.76 129.24) (stroke (width 0.1) (type default)) (layer "F.SilkS"))
 (gr_line (start 264.98 124.74) (end 269.24 124.74) (stroke (width 0.1) (type default)) (layer "F.SilkS"))
 (gr_line (start 264.99 35.96) (end 269.63 35.96) (stroke (width 0.1) (type default)) (layer "F.SilkS"))
 (gr_line (start 266.99 29.86) (end 266.99 44.38) (stroke (width 0.1) (type default)) (layer "F.SilkS"))
 (gr_line (start 266.99 128.3) (end 266.99 120.08) (stroke (width 0.1) (type default)) (layer "F.SilkS"))
 (gr_line (start 269.99 129.24) (end 269.99 121.25) (stroke (width 0.1) (type default)) (layer "F.SilkS"))
 (gr_line (start 270 30.17) (end 268.55 30.17) (stroke (width 0.1) (type default)) (layer "F.SilkS"))
 (gr_line (start 270 30.17) (end 270 32.42) (stroke (width 0.1) (type default)) (layer "F.SilkS"))
 (gr_line (start 270 40.82) (end 270 38.41) (stroke (width 0.1) (type default)) (layer "F.SilkS"))
 (gr_line (start 270 119.72) (end 270 117.63) (stroke (width 0.1) (type default)) (layer "F.SilkS"))
 (gr_rect (start 119.68 28.96) (end 269.99 129.24) (stroke (width 0.05) (type default)) (fill no) (layer "Edge.Cuts"))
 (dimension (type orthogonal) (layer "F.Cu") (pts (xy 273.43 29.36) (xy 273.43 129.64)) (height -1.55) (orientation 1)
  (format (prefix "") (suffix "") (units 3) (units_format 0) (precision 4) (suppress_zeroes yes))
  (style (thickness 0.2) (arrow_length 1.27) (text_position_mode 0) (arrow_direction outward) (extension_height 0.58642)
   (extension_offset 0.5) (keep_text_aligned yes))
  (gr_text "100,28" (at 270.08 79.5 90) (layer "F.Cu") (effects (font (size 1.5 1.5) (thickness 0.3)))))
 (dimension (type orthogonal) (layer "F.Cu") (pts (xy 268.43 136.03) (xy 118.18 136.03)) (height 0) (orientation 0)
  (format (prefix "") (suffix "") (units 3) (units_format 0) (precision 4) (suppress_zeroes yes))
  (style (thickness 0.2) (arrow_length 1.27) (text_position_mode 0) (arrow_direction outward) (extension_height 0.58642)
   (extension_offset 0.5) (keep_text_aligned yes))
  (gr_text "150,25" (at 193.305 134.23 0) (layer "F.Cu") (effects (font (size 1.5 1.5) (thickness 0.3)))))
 (segment (start 266.57 113.18) (end 266.45 116.57) (width 0.2) (layer "F.Cu") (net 32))
 (segment (start 264.99 119.71) (end 262.45 119.71) (width 0.2) (layer "F.Cu") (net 32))
 (segment (start 266.45 116.57) (end 264.99 117.17) (width 0.2) (layer "F.Cu") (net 32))
 (segment (start 264.99 112.09) (end 266.57 113.18) (width 0.2) (layer "F.Cu") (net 32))
 (segment (start 262.45 119.71) (end 259.91 119.71) (width 0.2) (layer "F.Cu") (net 32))
 (segment (start 264.99 117.17) (end 264.99 119.71) (width 0.2) (layer "F.Cu") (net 32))
 (segment (start 264.99 40.97) (end 262.45 40.97) (width 0.2) (layer "F.Cu") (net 1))
 (segment (start 262.45 40.97) (end 259.91 40.97) (width 0.2) (layer "F.Cu") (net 1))
 (segment (start 259.91 40.97) (end 256.17 40.97) (width 0.2) (layer "F.Cu") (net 1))
 (segment (start 264.99 63.83) (end 263.08 65.06) (width 0.2) (layer "F.Cu") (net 71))
 (segment (start 263.08 65.06) (end 256.61 65.06) (width 0.2) (layer "F.Cu") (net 71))
 (segment (start 263.08 90.31) (end 257.38 90.4) (width 0.2) (layer "F.Cu") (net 81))
 (segment (start 264.99 89.23) (end 263.08 90.31) (width 0.2) (layer "F.Cu") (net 81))
 (segment (start 259.91 94.31) (end 257.47 94.37) (width 0.2) (layer "F.Cu") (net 22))
 (segment (start 263.14 103.12) (end 257.41 103.08) (width 0.2) (layer "F.Cu") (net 87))
 (segment (start 264.99 104.47) (end 263.14 103.12) (width 0.2) (layer "F.Cu") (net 87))
 (segment (start 263.03 60.04) (end 256.3 60.09) (width 0.2) (layer "F.Cu") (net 69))
 (segment (start 264.99 58.75) (end 263.03 60.04) (width 0.2) (layer "F.Cu") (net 69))
 (segment (start 259.91 96.85) (end 257.33 96.95) (width 0.2) (layer "F.Cu") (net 23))
 (segment (start 259.91 43.51) (end 256.21 43.52) (width 0.2) (layer "F.Cu") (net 2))
 (segment (start 264.99 96.85) (end 263.04 95.59) (width 0.2) (layer "F.Cu") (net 84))
 (segment (start 263.04 95.59) (end 257.56 95.64) (width 0.2) (layer "F.Cu") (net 84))
 (segment (start 236.74 47.12) (end 251.63 47.08) (width 0.2) (layer "F.Cu") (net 7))
 (segment (start 263.13 75.24) (end 256.82 75.24) (width 0.2) (layer "F.Cu") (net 75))
 (segment (start 264.99 73.99) (end 263.13 75.24) (width 0.2) (layer "F.Cu") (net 75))
 (segment (start 259.91 66.37) (end 256.58 66.36) (width 0.2) (layer "F.Cu") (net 11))
 (segment (start 263.08 100.55) (end 257.33 100.5) (width 0.2) (layer "F.Cu") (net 86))
 (segment (start 264.99 101.93) (end 263.08 100.55) (width 0.2) (layer "F.Cu") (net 86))
 (segment (start 263.11 67.66) (end 256.55 67.66) (width 0.2) (layer "F.Cu") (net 72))
 (segment (start 264.99 66.37) (end 263.11 67.66) (width 0.2) (layer "F.Cu") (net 72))
 (segment (start 259.91 61.29) (end 256.39 61.29) (width 0.2) (layer "F.Cu") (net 9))
 (segment (start 263.18 85.44) (end 257.05 85.35) (width 0.2) (layer "F.Cu") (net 79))
 (segment (start 264.99 84.15) (end 263.18 85.44) (width 0.2) (layer "F.Cu") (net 79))
 (segment (start 259.91 114.63) (end 257.37 114.5) (width 0.2) (layer "F.Cu") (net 30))
 (segment (start 259.91 91.77) (end 257.42 91.76) (width 0.2) (layer "F.Cu") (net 21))
 (segment (start 259.91 86.69) (end 257.14 86.75) (width 0.2) (layer "F.Cu") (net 19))
 (segment (start 259.91 117.17) (end 257.45 117.08) (width 0.2) (layer "F.Cu") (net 31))
 (segment (start 262.98 62.63) (end 256.42 62.59) (width 0.2) (layer "F.Cu") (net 70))
 (segment (start 264.99 61.29) (end 262.98 62.63) (width 0.2) (layer "F.Cu") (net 70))
 (segment (start 259.91 73.99) (end 256.7 73.92) (width 0.2) (layer "F.Cu") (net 14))
 (segment (start 264.99 79.07) (end 263.13 80.35) (width 0.2) (layer "F.Cu") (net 77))
 (segment (start 263.13 80.35) (end 257.01 80.35) (width 0.2) (layer "F.Cu") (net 77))
 (segment (start 263.21 77.81) (end 256.97 77.85) (width 0.2) (layer "F.Cu") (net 76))
 (segment (start 264.99 76.53) (end 263.21 77.81) (width 0.2) (layer "F.Cu") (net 76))
 (segment (start 263.08 92.92) (end 257.47 92.97) (width 0.2) (layer "F.Cu") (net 83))
 (segment (start 264.99 94.31) (end 263.08 92.92) (width 0.2) (layer "F.Cu") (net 83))
 (segment (start 259.91 112.09) (end 257.41 111.93) (width 0.2) (layer "F.Cu") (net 29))
 (segment (start 259.91 48.59) (end 256.27 48.63) (width 0.2) (layer "F.Cu") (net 4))
 (segment (start 259.91 104.47) (end 257.37 104.56) (width 0.2) (layer "F.Cu") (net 26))
 (segment (start 259.91 109.55) (end 257.33 109.55) (width 0.2) (layer "F.Cu") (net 28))
 (segment (start 259.91 63.83) (end 256.48 63.83) (width 0.2) (layer "F.Cu") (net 10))
 (segment (start 264.99 46.05) (end 263.41 47.21) (width 0.2) (layer "F.Cu") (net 64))
 (segment (start 263.41 47.21) (end 256.26 47.26) (width 0.2) (layer "F.Cu") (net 64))
 (segment (start 259.91 107.01) (end 257.37 107.1) (width 0.2) (layer "F.Cu") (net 27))
 (segment (start 264.99 43.51) (end 263.39 44.79) (width 0.2) (layer "F.Cu") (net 63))
 (segment (start 263.39 44.79) (end 256.29 44.71) (width 0.2) (layer "F.Cu") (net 63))
 (segment (start 259.91 46.05) (end 256.23 46.02) (width 0.2) (layer "F.Cu") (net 3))
 (segment (start 264.99 81.61) (end 263.17 83) (width 0.2) (layer "F.Cu") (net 78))
 (segment (start 263.17 83) (end 256.97 82.96) (width 0.2) (layer "F.Cu") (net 78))
 (segment (start 259.91 101.93) (end 257.33 101.95) (width 0.2) (layer "F.Cu") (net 25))
 (segment (start 259.91 99.39) (end 257.38 99.38) (width 0.2) (layer "F.Cu") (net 24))
 (segment (start 259.91 76.53) (end 256.9 76.57) (width 0.2) (layer "F.Cu") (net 15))
 (segment (start 259.91 51.13) (end 256.24 51.16) (width 0.2) (layer "F.Cu") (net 5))
 (segment (start 259.91 53.67) (end 256.21 53.66) (width 0.2) (layer "F.Cu") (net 6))
 (segment (start 259.91 68.91) (end 256.58 68.9) (width 0.2) (layer "F.Cu") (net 12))
 (segment (start 259.91 89.23) (end 257.24 89.28) (width 0.2) (layer "F.Cu") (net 20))
 (segment (start 259.91 81.61) (end 257.01 81.63) (width 0.2) (layer "F.Cu") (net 17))
 (segment (start 259.91 71.45) (end 256.66 71.5) (width 0.2) (layer "F.Cu") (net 13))
 (segment (start 259.91 79.07) (end 256.97 79.02) (width 0.2) (layer "F.Cu") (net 16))
 (segment (start 263.08 98.12) (end 257.42 97.98) (width 0.2) (layer "F.Cu") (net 85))
 (segment (start 264.99 99.39) (end 263.08 98.12) (width 0.2) (layer "F.Cu") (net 85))
 (segment (start 263.18 105.85) (end 257.48 105.81) (width 0.2) (layer "F.Cu") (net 88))
 (segment (start 264.99 107.01) (end 263.18 105.85) (width 0.2) (layer "F.Cu") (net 88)))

